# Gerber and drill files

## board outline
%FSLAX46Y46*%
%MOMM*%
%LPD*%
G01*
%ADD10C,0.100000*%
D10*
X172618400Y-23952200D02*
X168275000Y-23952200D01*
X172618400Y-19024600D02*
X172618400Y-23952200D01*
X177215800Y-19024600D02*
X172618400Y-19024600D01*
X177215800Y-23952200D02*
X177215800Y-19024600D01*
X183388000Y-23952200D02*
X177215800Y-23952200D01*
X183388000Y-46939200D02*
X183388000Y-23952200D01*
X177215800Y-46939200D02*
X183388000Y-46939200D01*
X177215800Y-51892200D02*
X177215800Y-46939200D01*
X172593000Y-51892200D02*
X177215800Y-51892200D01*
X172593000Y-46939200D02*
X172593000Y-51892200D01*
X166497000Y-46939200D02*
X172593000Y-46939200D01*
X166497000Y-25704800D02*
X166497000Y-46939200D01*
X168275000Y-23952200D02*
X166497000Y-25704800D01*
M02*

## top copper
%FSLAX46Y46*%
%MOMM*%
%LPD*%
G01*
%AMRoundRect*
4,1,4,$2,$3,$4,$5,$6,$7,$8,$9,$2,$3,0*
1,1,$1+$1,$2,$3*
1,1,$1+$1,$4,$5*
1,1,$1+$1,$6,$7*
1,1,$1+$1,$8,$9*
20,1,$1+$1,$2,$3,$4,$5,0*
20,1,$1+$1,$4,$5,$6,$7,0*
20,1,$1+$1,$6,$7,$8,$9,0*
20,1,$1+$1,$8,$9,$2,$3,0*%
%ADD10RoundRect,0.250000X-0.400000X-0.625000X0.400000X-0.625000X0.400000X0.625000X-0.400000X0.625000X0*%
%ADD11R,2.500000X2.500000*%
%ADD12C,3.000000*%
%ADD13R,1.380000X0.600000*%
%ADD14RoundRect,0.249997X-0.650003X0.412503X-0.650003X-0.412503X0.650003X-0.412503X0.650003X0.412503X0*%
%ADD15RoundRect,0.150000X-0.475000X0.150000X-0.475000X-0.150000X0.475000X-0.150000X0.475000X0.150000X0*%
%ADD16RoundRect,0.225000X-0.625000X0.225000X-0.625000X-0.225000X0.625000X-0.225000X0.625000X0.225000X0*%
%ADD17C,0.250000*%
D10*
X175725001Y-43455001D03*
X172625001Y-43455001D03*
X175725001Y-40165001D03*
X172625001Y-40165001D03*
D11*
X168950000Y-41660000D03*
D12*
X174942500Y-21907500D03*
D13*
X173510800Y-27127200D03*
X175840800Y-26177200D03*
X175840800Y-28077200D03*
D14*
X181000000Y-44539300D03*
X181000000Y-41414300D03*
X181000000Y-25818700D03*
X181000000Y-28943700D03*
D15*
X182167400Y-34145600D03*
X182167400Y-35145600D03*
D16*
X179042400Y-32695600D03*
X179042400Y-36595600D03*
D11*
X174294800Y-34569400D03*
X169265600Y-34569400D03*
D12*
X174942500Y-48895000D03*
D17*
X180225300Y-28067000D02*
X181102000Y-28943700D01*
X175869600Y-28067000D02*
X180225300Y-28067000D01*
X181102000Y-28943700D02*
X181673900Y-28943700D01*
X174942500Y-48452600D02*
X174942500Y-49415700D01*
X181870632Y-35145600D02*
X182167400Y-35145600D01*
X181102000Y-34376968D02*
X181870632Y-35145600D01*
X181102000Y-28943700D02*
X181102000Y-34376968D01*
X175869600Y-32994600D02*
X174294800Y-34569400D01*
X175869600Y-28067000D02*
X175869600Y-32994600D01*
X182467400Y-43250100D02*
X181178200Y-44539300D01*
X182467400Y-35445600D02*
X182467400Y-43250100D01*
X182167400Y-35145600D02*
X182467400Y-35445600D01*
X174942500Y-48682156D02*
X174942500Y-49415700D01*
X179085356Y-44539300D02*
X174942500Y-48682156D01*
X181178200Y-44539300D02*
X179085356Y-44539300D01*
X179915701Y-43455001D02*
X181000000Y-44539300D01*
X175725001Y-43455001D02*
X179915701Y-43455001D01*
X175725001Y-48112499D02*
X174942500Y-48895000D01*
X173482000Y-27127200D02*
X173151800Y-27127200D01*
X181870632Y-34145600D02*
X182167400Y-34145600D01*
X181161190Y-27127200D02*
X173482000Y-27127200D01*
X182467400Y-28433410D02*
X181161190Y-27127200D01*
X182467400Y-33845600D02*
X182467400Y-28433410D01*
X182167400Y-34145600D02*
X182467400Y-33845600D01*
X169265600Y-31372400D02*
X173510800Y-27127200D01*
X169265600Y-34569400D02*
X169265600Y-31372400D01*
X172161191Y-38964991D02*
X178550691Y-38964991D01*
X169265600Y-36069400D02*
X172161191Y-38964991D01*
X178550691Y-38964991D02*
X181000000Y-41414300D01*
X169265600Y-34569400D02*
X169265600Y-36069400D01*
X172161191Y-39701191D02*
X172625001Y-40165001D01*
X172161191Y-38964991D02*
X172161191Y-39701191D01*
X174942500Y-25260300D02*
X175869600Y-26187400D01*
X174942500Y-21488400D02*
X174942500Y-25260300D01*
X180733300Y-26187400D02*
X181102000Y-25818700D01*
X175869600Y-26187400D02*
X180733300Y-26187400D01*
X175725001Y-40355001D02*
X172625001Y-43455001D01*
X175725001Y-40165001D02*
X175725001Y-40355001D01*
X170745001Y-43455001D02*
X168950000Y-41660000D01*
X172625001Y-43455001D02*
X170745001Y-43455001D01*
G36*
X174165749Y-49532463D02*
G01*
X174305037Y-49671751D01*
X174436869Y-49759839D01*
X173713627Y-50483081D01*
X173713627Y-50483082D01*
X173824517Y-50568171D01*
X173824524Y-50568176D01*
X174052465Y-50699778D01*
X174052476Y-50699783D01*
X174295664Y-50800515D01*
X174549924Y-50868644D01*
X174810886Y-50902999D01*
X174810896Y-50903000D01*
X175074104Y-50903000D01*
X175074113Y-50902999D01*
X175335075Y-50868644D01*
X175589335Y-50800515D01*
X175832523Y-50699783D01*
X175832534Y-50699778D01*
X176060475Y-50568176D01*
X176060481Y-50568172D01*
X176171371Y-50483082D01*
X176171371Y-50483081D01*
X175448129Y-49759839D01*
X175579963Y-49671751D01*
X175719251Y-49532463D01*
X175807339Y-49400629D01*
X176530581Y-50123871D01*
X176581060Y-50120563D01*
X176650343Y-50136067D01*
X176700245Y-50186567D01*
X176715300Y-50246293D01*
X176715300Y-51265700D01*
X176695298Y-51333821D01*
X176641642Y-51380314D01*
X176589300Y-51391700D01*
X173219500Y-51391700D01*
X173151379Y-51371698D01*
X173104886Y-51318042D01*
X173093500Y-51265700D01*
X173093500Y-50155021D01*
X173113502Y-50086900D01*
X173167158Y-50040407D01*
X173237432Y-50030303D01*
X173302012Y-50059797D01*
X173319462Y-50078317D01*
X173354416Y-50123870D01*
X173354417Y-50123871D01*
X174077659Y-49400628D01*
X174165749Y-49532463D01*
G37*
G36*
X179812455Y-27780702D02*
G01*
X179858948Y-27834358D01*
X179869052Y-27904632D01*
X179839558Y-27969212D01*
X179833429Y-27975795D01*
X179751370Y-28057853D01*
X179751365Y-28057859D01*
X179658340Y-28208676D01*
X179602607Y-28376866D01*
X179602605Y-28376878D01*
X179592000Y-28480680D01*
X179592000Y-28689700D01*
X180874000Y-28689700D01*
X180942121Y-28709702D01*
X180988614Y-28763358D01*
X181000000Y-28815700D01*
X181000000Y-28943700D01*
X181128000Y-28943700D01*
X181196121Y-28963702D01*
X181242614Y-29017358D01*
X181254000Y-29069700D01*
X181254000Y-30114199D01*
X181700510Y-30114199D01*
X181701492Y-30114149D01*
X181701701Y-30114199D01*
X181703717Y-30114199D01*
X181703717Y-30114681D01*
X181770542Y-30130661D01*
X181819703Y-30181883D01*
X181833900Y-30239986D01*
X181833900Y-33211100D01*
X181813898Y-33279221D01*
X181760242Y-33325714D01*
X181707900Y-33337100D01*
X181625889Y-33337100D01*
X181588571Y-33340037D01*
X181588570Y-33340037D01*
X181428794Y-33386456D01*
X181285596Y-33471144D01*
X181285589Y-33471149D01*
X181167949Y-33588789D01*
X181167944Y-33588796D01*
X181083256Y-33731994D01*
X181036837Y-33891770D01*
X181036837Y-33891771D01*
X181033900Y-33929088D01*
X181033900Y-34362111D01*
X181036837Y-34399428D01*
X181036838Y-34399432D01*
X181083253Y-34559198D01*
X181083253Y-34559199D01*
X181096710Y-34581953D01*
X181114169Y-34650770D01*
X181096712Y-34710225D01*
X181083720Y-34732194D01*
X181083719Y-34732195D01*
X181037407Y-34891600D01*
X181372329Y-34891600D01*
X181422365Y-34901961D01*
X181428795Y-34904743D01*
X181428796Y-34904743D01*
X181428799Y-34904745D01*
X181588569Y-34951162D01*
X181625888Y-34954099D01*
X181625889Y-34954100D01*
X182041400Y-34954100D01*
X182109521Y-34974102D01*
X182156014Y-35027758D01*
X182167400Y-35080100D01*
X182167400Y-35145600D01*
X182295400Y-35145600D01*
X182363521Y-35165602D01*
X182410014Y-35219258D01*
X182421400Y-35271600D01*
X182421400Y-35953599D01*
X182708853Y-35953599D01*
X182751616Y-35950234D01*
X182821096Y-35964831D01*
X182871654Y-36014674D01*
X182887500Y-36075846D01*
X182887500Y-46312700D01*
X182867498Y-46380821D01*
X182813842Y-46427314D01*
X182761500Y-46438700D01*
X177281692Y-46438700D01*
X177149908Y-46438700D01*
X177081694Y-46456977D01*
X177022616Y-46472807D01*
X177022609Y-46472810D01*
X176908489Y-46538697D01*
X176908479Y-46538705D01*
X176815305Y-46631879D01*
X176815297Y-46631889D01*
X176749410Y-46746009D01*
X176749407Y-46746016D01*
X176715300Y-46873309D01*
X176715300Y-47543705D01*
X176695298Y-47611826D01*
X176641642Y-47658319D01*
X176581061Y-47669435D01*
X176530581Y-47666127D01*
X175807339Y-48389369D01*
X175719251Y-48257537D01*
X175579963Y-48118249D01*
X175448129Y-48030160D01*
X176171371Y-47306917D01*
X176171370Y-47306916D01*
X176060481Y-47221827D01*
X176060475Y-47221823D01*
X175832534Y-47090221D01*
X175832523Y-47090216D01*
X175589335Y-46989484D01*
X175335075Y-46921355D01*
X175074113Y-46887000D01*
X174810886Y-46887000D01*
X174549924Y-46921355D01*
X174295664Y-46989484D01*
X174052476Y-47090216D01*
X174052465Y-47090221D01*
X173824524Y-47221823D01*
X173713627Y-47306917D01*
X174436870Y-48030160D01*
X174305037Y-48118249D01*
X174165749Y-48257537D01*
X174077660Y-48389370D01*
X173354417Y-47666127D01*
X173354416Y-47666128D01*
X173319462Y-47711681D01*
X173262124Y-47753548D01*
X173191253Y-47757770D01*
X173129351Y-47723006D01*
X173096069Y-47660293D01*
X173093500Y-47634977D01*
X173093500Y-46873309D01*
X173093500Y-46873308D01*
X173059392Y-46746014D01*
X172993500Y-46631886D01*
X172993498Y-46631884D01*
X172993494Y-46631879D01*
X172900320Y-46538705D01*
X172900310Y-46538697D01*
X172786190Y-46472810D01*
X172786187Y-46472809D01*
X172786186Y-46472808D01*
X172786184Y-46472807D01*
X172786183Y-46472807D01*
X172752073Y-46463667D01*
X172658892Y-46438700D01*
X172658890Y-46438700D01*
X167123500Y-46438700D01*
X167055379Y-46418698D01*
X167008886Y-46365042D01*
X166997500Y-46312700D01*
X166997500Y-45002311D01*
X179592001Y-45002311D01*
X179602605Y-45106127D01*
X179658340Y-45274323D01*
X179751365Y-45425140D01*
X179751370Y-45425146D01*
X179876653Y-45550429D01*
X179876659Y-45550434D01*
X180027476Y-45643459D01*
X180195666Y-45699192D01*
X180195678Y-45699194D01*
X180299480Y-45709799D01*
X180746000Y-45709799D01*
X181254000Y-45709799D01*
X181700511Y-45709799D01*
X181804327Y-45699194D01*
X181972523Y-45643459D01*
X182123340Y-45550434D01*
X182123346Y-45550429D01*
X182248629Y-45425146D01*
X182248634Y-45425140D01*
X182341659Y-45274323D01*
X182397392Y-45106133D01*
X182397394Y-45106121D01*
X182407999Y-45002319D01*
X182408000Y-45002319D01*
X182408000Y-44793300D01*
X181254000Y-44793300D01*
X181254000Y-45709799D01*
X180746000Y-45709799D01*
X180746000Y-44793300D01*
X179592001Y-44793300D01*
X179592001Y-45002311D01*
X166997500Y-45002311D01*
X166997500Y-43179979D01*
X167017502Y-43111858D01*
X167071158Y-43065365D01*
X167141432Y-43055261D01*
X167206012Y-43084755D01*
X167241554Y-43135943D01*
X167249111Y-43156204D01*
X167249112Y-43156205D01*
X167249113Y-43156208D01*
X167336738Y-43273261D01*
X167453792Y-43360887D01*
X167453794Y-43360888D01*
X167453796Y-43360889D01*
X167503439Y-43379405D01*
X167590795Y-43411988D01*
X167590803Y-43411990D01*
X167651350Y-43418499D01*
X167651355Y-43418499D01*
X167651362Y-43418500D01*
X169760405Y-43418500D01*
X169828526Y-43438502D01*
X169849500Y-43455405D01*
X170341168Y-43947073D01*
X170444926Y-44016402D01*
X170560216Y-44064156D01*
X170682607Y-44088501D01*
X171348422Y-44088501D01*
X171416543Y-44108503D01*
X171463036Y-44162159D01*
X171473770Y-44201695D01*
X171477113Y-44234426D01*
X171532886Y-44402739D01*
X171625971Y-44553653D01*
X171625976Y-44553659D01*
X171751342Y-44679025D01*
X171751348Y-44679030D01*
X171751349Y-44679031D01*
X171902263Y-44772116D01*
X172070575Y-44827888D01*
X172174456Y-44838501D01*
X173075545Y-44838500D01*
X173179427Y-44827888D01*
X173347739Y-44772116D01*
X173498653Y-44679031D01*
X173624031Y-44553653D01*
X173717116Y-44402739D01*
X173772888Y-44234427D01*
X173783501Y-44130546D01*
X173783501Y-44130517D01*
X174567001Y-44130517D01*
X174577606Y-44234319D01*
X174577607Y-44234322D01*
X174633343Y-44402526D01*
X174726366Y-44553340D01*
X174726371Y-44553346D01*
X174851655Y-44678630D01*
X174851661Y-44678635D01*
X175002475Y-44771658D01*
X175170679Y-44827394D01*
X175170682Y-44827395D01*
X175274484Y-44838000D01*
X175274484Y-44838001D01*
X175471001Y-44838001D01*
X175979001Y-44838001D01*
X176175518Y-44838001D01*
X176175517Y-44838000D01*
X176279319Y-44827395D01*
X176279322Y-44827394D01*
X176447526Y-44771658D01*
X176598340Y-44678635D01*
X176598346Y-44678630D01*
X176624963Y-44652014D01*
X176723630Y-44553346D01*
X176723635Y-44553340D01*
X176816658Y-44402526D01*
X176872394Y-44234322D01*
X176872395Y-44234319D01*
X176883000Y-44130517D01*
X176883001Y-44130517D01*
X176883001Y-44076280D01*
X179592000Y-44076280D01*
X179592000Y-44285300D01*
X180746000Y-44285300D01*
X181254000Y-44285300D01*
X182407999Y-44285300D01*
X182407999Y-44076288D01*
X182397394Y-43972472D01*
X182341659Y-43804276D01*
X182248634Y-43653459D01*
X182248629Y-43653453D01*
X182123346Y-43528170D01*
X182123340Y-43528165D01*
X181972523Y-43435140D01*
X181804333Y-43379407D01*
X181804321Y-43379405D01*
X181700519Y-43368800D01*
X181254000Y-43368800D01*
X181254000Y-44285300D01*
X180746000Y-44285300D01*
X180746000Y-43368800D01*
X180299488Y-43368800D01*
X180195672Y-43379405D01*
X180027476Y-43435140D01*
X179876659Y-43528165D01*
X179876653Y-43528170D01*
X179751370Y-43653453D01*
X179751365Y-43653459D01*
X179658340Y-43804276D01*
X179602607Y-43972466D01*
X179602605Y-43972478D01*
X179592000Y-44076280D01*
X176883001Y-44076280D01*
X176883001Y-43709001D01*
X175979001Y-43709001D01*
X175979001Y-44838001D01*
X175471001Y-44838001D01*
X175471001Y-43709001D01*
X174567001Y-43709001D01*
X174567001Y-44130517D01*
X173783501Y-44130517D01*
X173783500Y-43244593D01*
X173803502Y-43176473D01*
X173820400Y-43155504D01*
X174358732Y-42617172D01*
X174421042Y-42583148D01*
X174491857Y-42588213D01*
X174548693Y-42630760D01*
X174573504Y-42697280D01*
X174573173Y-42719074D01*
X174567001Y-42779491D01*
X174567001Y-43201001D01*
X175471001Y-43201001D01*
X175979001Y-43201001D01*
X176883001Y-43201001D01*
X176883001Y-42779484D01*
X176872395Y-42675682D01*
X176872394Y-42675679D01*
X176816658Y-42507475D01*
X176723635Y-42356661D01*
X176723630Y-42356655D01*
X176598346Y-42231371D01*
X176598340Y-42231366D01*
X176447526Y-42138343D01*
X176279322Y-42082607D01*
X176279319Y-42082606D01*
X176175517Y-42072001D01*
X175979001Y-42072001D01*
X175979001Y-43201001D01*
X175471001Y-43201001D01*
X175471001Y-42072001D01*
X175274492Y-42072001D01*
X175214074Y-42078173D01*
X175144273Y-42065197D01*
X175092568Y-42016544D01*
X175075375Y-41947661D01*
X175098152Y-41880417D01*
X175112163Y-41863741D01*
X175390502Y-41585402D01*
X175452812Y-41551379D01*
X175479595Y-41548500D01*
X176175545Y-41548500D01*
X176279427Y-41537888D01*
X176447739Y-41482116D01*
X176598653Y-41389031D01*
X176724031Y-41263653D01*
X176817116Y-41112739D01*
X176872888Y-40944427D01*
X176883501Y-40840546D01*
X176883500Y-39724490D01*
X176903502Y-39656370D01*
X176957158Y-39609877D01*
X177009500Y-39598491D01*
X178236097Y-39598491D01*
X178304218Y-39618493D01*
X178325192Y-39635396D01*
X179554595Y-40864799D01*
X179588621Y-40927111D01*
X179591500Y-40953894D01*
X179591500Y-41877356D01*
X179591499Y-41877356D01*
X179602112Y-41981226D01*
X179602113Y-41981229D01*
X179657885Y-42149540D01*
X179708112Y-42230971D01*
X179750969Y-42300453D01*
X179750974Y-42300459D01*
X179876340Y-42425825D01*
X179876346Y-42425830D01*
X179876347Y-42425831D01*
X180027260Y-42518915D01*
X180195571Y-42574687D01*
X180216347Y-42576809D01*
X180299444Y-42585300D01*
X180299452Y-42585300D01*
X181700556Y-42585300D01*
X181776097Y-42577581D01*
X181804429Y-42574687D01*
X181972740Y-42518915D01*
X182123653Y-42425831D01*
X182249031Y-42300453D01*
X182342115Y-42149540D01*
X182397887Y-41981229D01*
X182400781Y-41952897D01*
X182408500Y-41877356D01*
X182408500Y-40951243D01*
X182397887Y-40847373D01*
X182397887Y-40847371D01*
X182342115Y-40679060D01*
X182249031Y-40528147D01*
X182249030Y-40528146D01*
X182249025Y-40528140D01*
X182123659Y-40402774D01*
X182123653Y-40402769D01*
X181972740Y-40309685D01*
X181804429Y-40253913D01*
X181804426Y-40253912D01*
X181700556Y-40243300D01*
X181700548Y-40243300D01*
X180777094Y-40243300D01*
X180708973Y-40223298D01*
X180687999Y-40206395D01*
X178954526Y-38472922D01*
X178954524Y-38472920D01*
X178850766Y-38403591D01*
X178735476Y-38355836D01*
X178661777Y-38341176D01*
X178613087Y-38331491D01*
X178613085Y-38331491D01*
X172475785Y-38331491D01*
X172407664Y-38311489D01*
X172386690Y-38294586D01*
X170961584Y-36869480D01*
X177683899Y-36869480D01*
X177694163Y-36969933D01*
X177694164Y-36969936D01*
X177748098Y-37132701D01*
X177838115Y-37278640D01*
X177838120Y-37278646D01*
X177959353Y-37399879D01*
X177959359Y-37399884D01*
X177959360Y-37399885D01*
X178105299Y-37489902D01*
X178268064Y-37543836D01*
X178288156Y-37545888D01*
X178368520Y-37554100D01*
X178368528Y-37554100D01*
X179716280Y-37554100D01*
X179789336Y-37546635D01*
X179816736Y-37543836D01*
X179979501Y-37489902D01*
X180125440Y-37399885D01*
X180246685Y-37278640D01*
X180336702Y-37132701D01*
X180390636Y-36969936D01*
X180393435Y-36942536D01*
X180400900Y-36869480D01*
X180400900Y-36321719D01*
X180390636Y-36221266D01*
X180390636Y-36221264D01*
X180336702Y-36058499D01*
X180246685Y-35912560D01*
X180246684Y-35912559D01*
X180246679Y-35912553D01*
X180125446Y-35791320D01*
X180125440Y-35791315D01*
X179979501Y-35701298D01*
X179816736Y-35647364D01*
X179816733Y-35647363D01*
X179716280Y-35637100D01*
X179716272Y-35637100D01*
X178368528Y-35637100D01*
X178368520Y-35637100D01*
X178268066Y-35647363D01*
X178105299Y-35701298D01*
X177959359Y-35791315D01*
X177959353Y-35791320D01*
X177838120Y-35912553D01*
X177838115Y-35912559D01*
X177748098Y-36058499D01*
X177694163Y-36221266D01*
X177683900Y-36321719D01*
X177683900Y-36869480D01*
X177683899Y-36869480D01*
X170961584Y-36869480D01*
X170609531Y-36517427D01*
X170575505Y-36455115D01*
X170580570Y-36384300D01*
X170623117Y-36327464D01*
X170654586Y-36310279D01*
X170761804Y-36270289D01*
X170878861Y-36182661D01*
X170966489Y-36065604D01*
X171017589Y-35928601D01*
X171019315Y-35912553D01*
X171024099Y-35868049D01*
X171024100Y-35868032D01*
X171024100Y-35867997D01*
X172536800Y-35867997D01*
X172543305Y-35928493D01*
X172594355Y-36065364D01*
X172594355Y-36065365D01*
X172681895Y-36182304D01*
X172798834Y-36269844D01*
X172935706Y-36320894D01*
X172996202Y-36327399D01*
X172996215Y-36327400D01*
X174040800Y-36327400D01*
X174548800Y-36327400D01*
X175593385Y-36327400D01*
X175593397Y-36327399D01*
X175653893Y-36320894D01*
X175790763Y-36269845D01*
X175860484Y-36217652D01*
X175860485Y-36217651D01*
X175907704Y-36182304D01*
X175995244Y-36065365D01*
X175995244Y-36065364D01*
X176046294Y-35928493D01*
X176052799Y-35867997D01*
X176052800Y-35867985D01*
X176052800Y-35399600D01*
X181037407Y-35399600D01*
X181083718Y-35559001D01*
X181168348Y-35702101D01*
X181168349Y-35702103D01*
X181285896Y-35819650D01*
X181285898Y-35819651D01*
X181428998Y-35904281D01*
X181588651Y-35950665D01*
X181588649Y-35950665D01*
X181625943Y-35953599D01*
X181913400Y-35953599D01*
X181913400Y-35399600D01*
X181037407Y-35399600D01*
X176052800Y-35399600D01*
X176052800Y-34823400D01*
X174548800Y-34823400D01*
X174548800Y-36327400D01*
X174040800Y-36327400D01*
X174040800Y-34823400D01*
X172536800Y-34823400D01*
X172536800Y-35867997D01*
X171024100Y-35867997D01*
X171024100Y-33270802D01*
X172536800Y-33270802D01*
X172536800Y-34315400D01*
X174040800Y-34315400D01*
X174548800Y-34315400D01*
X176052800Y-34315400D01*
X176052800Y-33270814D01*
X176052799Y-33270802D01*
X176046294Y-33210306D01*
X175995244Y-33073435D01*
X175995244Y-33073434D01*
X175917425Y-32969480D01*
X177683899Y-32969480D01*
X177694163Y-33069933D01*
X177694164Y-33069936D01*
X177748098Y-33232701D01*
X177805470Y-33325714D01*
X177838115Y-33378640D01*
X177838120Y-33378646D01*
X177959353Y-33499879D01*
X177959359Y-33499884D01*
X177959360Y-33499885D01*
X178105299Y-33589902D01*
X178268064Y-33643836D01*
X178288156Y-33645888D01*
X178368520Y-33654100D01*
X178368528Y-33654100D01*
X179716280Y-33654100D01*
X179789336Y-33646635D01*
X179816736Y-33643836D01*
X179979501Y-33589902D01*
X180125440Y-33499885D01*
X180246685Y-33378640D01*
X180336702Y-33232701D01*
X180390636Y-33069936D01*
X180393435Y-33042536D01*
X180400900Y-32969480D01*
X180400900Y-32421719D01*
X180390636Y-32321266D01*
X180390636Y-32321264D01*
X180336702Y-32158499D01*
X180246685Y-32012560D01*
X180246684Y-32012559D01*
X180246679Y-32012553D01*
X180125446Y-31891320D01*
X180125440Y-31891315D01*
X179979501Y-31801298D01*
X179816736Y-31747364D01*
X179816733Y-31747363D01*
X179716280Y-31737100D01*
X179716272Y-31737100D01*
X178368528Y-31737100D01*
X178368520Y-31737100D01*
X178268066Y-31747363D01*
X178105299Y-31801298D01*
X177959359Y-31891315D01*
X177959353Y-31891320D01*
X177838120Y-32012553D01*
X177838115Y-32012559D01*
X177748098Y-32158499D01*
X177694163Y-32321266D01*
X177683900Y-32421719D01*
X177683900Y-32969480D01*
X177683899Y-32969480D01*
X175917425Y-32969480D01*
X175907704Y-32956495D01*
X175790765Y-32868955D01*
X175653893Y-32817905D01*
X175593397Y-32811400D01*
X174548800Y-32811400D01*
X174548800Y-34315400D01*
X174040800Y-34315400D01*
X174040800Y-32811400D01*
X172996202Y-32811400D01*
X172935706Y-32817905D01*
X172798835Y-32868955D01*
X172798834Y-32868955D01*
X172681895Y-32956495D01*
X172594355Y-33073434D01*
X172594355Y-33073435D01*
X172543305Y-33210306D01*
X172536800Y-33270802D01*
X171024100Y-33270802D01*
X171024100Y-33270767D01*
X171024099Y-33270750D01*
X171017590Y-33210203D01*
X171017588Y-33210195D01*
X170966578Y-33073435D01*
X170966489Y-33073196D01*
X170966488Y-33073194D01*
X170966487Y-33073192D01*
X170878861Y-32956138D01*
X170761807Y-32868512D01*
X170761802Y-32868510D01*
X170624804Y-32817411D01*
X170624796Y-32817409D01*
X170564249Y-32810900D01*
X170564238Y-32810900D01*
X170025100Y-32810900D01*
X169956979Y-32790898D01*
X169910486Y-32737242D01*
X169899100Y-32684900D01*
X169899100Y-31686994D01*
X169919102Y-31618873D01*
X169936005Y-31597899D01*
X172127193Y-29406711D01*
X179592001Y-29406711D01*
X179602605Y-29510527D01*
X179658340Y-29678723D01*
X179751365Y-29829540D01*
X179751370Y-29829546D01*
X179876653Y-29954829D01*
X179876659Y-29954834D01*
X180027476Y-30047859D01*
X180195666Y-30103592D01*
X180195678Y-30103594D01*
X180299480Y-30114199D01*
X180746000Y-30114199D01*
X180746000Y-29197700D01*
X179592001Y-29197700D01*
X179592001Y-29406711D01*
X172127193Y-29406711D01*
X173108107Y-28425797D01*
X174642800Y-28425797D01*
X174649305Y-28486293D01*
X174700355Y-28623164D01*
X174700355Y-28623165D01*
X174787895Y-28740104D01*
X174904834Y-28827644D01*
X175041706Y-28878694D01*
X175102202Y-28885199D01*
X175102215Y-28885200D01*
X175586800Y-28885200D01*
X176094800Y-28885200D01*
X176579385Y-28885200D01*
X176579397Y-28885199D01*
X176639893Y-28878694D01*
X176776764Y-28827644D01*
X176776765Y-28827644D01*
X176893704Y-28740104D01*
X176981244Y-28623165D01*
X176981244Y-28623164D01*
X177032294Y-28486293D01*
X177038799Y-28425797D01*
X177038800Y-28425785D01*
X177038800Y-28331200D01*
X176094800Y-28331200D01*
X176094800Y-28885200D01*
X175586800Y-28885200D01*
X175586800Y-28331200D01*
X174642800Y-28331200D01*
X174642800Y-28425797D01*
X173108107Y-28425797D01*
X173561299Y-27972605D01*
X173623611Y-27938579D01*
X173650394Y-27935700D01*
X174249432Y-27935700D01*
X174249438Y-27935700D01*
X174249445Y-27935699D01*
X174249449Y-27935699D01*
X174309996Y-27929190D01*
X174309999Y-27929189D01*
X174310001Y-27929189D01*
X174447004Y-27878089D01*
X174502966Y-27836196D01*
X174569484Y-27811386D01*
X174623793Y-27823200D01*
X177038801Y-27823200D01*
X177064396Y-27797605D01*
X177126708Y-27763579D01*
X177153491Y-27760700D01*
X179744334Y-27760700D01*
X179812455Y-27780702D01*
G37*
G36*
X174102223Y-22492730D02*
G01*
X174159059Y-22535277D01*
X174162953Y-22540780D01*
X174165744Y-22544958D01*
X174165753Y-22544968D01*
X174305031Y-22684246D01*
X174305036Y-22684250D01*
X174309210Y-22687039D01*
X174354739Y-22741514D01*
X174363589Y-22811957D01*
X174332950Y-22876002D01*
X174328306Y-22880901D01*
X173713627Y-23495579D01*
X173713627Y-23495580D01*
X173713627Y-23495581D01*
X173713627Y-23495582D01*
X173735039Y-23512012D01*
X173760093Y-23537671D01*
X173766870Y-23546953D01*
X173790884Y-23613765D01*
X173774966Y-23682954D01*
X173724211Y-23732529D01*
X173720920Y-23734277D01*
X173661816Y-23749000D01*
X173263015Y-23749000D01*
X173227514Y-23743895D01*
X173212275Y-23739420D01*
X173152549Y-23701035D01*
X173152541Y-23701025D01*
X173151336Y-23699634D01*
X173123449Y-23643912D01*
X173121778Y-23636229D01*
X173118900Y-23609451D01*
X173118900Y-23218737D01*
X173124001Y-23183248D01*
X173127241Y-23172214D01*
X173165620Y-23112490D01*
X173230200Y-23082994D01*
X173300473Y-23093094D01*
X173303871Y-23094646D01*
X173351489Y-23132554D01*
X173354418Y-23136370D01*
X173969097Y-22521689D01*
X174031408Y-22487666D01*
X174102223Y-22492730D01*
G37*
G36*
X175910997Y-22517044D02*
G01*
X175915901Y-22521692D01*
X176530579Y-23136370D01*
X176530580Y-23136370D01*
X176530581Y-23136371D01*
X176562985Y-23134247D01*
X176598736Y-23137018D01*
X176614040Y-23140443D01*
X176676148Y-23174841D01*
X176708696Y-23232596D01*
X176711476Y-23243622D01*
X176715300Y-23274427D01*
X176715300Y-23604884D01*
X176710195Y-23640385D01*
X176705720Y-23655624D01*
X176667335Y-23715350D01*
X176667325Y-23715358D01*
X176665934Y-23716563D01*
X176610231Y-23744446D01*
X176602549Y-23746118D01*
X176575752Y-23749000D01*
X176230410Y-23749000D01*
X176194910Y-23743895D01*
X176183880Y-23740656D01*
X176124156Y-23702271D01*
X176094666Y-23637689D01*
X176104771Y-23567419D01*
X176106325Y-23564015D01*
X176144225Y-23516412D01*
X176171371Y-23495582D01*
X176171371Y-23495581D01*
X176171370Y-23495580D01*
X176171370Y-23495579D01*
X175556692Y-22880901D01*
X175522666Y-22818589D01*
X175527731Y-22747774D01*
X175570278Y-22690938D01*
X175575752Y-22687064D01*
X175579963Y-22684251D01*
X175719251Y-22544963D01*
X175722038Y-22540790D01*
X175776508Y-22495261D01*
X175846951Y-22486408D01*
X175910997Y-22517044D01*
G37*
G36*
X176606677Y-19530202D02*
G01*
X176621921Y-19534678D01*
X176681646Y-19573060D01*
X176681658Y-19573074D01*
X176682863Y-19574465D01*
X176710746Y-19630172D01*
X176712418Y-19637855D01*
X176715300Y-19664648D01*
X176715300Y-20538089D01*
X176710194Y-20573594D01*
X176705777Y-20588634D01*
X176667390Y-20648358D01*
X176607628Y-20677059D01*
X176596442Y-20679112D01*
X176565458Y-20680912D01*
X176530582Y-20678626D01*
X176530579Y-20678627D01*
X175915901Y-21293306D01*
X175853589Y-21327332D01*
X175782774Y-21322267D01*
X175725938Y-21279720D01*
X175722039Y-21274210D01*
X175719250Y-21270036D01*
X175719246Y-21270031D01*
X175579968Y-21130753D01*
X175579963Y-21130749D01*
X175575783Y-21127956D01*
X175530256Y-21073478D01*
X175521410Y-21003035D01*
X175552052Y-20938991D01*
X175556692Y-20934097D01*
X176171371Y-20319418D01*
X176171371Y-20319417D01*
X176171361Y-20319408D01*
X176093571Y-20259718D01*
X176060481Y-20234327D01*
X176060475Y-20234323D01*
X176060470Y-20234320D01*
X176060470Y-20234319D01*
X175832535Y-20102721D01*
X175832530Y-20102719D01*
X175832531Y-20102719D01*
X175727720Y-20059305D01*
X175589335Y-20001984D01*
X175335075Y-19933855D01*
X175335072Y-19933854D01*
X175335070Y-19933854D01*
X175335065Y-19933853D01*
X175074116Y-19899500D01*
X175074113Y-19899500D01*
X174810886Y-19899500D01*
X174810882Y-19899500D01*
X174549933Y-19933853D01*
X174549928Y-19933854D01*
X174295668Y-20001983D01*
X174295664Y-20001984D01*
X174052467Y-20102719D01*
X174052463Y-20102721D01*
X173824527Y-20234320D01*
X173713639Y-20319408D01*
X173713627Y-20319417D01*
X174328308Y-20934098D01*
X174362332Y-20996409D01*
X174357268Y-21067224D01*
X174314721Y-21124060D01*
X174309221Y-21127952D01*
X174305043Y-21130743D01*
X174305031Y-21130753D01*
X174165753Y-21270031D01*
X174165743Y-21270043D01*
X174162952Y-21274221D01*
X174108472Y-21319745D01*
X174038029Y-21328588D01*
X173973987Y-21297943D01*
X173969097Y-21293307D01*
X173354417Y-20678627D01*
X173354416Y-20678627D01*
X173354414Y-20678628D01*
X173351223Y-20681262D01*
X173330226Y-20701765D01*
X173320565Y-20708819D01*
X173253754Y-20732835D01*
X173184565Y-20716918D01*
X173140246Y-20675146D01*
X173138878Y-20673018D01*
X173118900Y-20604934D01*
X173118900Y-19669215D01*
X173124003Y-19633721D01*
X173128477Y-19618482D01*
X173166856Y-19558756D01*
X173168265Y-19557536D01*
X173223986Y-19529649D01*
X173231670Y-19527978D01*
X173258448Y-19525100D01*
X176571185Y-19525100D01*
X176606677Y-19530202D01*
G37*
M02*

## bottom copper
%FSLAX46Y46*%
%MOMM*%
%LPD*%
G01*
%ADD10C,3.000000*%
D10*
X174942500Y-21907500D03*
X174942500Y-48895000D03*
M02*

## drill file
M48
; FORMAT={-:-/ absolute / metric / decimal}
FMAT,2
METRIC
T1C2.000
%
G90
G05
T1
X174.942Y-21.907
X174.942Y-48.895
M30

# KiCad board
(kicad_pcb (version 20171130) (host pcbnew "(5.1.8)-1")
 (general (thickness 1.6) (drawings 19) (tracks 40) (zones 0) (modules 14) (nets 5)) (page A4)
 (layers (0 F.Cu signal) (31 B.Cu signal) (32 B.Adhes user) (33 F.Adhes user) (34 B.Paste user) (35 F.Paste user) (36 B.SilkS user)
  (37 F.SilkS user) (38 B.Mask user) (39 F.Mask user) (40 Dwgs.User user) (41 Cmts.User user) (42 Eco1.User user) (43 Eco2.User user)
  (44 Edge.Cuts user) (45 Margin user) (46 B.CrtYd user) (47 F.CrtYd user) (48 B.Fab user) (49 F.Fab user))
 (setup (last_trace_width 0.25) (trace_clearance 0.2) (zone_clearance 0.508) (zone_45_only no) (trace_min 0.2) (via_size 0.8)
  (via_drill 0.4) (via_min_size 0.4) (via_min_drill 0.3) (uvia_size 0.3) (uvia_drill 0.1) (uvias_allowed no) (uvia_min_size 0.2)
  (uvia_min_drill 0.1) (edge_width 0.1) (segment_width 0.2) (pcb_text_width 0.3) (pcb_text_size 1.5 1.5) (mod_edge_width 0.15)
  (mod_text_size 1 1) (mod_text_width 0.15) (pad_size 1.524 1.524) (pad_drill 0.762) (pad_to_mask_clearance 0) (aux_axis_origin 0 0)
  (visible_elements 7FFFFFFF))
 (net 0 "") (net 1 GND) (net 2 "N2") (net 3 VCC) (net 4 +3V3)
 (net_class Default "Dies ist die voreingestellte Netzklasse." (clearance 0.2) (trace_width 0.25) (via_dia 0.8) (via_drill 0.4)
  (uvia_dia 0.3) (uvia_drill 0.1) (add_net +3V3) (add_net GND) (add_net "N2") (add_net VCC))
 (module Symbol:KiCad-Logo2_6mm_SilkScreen (layer B.Cu) (at 169.7 35.36 270)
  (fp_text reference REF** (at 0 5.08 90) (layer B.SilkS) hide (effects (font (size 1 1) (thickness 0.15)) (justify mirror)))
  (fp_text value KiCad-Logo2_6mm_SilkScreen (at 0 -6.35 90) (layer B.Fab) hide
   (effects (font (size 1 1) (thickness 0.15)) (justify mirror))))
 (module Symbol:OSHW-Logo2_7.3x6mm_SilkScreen (layer B.Cu) (at 178.48 35.75 270)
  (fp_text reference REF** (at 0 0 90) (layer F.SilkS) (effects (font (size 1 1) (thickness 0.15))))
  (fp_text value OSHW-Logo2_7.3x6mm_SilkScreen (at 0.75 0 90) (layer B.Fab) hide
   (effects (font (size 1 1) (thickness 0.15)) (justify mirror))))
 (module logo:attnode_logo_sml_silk (layer F.Cu) (at 169.78 25.8)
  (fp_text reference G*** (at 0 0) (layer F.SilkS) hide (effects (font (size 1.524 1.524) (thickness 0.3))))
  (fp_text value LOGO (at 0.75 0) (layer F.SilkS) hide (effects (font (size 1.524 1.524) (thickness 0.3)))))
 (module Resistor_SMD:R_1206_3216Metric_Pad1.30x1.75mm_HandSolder (layer F.Cu) (at 174.175001 43.455001)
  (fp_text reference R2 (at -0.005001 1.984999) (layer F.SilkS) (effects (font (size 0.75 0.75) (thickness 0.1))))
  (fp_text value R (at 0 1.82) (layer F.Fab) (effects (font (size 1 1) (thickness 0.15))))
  (pad 2 smd roundrect (at 1.55 0) (size 1.3 1.75) (layers F.Cu F.Paste F.Mask) (roundrect_rratio 0.1923076923076923) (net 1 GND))
  (pad 1 smd roundrect (at -1.55 0) (size 1.3 1.75) (layers F.Cu F.Paste F.Mask) (roundrect_rratio 0.1923076923076923) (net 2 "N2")))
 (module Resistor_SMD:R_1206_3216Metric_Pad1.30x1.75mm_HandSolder (layer F.Cu) (at 174.175001 40.165001)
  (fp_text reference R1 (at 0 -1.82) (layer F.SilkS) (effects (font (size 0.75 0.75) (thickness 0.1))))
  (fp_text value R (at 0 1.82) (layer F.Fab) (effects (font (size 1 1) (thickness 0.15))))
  (pad 2 smd roundrect (at 1.55 0) (size 1.3 1.75) (layers F.Cu F.Paste F.Mask) (roundrect_rratio 0.1923076923076923) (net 2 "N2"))
  (pad 1 smd roundrect (at -1.55 0) (size 1.3 1.75) (layers F.Cu F.Paste F.Mask) (roundrect_rratio 0.1923076923076923) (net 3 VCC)))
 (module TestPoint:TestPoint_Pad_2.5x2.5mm (layer F.Cu) (at 168.95 41.66)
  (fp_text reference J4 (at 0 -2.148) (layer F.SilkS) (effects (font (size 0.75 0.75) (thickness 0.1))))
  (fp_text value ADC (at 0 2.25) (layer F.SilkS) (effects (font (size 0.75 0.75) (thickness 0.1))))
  (pad 1 smd rect (at 0 0) (size 2.5 2.5) (layers F.Cu F.Mask) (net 2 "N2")))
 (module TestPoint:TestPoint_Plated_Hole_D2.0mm (layer F.Cu) (at 174.9425 21.9075)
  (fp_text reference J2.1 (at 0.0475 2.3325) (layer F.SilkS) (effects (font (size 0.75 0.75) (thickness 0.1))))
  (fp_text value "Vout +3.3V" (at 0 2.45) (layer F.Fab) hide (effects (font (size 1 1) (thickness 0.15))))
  (pad 1 thru_hole circle (at 0 0) (size 3 3) (drill 2) (layers *.Cu *.Mask) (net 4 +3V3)))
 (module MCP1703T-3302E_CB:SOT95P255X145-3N (layer F.Cu) (at 174.6758 27.1272 180)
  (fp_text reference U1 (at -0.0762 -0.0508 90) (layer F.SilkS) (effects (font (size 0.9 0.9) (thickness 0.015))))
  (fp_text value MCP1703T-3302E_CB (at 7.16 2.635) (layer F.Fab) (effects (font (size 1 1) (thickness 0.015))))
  (pad 3 smd rect (at 1.165 0 180) (size 1.38 0.6) (layers F.Cu F.Paste F.Mask) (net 3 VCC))
  (pad 2 smd rect (at -1.165 0.95 180) (size 1.38 0.6) (layers F.Cu F.Paste F.Mask) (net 4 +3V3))
  (pad 1 smd rect (at -1.165 -0.95 180) (size 1.38 0.6) (layers F.Cu F.Paste F.Mask) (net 1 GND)))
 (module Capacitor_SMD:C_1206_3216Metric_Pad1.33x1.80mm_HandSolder (layer F.Cu) (at 181 42.9768 270)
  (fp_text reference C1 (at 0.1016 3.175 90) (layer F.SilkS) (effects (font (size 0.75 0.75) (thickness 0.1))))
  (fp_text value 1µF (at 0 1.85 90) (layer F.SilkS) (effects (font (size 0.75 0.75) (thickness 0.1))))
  (pad 2 smd roundrect (at 1.5625 0 270) (size 1.325 1.8) (layers F.Cu F.Paste F.Mask) (roundrect_rratio 0.1886769811320755) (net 1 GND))
  (pad 1 smd roundrect (at -1.5625 0 270) (size 1.325 1.8) (layers F.Cu F.Paste F.Mask) (roundrect_rratio 0.1886769811320755) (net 3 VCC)))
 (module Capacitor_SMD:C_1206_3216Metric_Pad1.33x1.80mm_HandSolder (layer F.Cu) (at 181 27.3812 270)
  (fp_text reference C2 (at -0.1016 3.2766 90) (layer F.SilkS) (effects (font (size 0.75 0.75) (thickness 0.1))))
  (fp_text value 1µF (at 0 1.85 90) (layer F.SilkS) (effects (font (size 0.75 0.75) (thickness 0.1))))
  (pad 1 smd roundrect (at -1.5625 0 270) (size 1.325 1.8) (layers F.Cu F.Paste F.Mask) (roundrect_rratio 0.1886769811320755) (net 4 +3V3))
  (pad 2 smd roundrect (at 1.5625 0 270) (size 1.325 1.8) (layers F.Cu F.Paste F.Mask) (roundrect_rratio 0.1886769811320755) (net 1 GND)))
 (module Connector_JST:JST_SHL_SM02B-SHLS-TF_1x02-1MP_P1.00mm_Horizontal (layer F.Cu) (at 180.4924 34.6456 270)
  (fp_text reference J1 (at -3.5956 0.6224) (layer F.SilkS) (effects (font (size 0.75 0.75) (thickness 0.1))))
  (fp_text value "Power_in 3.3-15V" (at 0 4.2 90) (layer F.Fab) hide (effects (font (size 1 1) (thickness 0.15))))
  (pad 1 smd roundrect (at -0.5 -1.675 270) (size 0.6 1.25) (layers F.Cu F.Paste F.Mask) (roundrect_rratio 0.25) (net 3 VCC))
  (pad 2 smd roundrect (at 0.5 -1.675 270) (size 0.6 1.25) (layers F.Cu F.Paste F.Mask) (roundrect_rratio 0.25) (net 1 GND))
  (pad MP smd roundrect (at -1.95 1.45 270) (size 0.9 1.7) (layers F.Cu F.Paste F.Mask) (roundrect_rratio 0.25))
  (pad MP smd roundrect (at 1.95 1.45 270) (size 0.9 1.7) (layers F.Cu F.Paste F.Mask) (roundrect_rratio 0.25)))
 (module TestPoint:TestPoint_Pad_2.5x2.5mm (layer F.Cu) (at 174.2948 34.5694)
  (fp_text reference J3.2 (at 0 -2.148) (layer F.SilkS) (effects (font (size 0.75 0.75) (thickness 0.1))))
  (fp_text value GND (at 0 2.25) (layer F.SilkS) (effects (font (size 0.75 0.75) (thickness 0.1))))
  (pad 1 smd rect (at 0 0) (size 2.5 2.5) (layers F.Cu F.Mask) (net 1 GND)))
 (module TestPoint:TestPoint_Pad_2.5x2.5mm (layer F.Cu) (at 169.2656 34.5694)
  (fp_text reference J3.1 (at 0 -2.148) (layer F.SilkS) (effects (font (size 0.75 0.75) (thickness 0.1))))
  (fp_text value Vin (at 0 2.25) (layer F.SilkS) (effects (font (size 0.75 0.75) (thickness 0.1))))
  (pad 1 smd rect (at 0 0) (size 2.5 2.5) (layers F.Cu F.Mask) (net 3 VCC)))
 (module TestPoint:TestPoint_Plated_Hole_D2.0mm (layer F.Cu) (at 174.9425 48.895)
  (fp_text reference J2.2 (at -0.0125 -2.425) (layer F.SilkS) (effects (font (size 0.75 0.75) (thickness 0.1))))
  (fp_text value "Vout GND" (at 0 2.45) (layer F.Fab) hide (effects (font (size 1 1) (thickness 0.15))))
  (pad 1 thru_hole circle (at 0 0) (size 3 3) (drill 2) (layers *.Cu *.Mask) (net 1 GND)))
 (gr_line (start 172.6184 23.9522) (end 168.275 23.9522) (layer Edge.Cuts) (width 0.1))
 (gr_line (start 172.6184 19.0246) (end 172.6184 23.9522) (layer Edge.Cuts) (width 0.1))
 (gr_line (start 177.2158 19.0246) (end 172.6184 19.0246) (layer Edge.Cuts) (width 0.1))
 (gr_line (start 177.2158 23.9522) (end 177.2158 19.0246) (layer Edge.Cuts) (width 0.1))
 (gr_line (start 183.388 23.9522) (end 177.2158 23.9522) (layer Edge.Cuts) (width 0.1))
 (gr_line (start 183.388 46.9392) (end 183.388 23.9522) (layer Edge.Cuts) (width 0.1))
 (gr_line (start 177.2158 46.9392) (end 183.388 46.9392) (layer Edge.Cuts) (width 0.1))
 (gr_line (start 177.2158 51.8922) (end 177.2158 46.9392) (layer Edge.Cuts) (width 0.1))
 (gr_line (start 172.593 51.8922) (end 177.2158 51.8922) (layer Edge.Cuts) (width 0.1))
 (gr_line (start 172.593 46.9392) (end 172.593 51.8922) (layer Edge.Cuts) (width 0.1))
 (gr_line (start 166.497 46.9392) (end 172.593 46.9392) (layer Edge.Cuts) (width 0.1))
 (gr_line (start 166.497 25.7048) (end 166.497 46.9392) (layer Edge.Cuts) (width 0.1))
 (gr_line (start 168.275 23.9522) (end 166.497 25.7048) (layer Edge.Cuts) (width 0.1))
 (segment (start 180.2253 28.067) (end 181.102 28.9437) (width 0.25) (layer F.Cu) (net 1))
 (segment (start 175.8696 28.067) (end 180.2253 28.067) (width 0.25) (layer F.Cu) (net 1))
 (segment (start 181.102 28.9437) (end 181.6739 28.9437) (width 0.25) (layer F.Cu) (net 1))
 (segment (start 174.9425 48.4526) (end 174.9425 49.4157) (width 0.25) (layer F.Cu) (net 1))
 (segment (start 181.870632 35.1456) (end 182.1674 35.1456) (width 0.25) (layer F.Cu) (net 1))
 (segment (start 181.102 34.376968) (end 181.870632 35.1456) (width 0.25) (layer F.Cu) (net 1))
 (segment (start 181.102 28.9437) (end 181.102 34.376968) (width 0.25) (layer F.Cu) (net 1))
 (segment (start 175.8696 32.9946) (end 174.2948 34.5694) (width 0.25) (layer F.Cu) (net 1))
 (segment (start 175.8696 28.067) (end 175.8696 32.9946) (width 0.25) (layer F.Cu) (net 1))
 (segment (start 182.4674 43.2501) (end 181.1782 44.5393) (width 0.25) (layer F.Cu) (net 1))
 (segment (start 182.4674 35.4456) (end 182.4674 43.2501) (width 0.25) (layer F.Cu) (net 1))
 (segment (start 182.1674 35.1456) (end 182.4674 35.4456) (width 0.25) (layer F.Cu) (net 1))
 (segment (start 174.9425 48.682156) (end 174.9425 49.4157) (width 0.25) (layer F.Cu) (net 1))
 (segment (start 179.085356 44.5393) (end 174.9425 48.682156) (width 0.25) (layer F.Cu) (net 1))
 (segment (start 181.1782 44.5393) (end 179.085356 44.5393) (width 0.25) (layer F.Cu) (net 1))
 (segment (start 179.915701 43.455001) (end 181 44.5393) (width 0.25) (layer F.Cu) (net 1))
 (segment (start 175.725001 43.455001) (end 179.915701 43.455001) (width 0.25) (layer F.Cu) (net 1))
 (segment (start 175.725001 48.112499) (end 174.9425 48.895) (width 0.25) (layer F.Cu) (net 1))
 (segment (start 173.482 27.1272) (end 173.1518 27.1272) (width 0.25) (layer F.Cu) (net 3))
 (segment (start 181.870632 34.1456) (end 182.1674 34.1456) (width 0.25) (layer F.Cu) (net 3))
 (segment (start 181.16119 27.1272) (end 173.482 27.1272) (width 0.25) (layer F.Cu) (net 3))
 (segment (start 182.4674 28.43341) (end 181.16119 27.1272) (width 0.25) (layer F.Cu) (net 3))
 (segment (start 182.4674 33.8456) (end 182.4674 28.43341) (width 0.25) (layer F.Cu) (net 3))
 (segment (start 182.1674 34.1456) (end 182.4674 33.8456) (width 0.25) (layer F.Cu) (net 3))
 (segment (start 169.2656 31.3724) (end 173.5108 27.1272) (width 0.25) (layer F.Cu) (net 3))
 (segment (start 169.2656 34.5694) (end 169.2656 31.3724) (width 0.25) (layer F.Cu) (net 3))
 (segment (start 172.161191 38.964991) (end 178.550691 38.964991) (width 0.25) (layer F.Cu) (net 3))
 (segment (start 169.2656 36.0694) (end 172.161191 38.964991) (width 0.25) (layer F.Cu) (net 3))
 (segment (start 178.550691 38.964991) (end 181 41.4143) (width 0.25) (layer F.Cu) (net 3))
 (segment (start 169.2656 34.5694) (end 169.2656 36.0694) (width 0.25) (layer F.Cu) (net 3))
 (segment (start 172.161191 39.701191) (end 172.625001 40.165001) (width 0.25) (layer F.Cu) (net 3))
 (segment (start 172.161191 38.964991) (end 172.161191 39.701191) (width 0.25) (layer F.Cu) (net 3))
 (segment (start 174.9425 25.2603) (end 175.8696 26.1874) (width 0.25) (layer F.Cu) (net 4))
 (segment (start 174.9425 21.4884) (end 174.9425 25.2603) (width 0.25) (layer F.Cu) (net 4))
 (segment (start 180.7333 26.1874) (end 181.102 25.8187) (width 0.25) (layer F.Cu) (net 4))
 (segment (start 175.8696 26.1874) (end 180.7333 26.1874) (width 0.25) (layer F.Cu) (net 4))
 (segment (start 175.725001 40.355001) (end 172.625001 43.455001) (width 0.25) (layer F.Cu) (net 2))
 (segment (start 175.725001 40.165001) (end 175.725001 40.355001) (width 0.25) (layer F.Cu) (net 2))
 (segment (start 170.745001 43.455001) (end 168.95 41.66) (width 0.25) (layer F.Cu) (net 2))
 (segment (start 172.625001 43.455001) (end 170.745001 43.455001) (width 0.25) (layer F.Cu) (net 2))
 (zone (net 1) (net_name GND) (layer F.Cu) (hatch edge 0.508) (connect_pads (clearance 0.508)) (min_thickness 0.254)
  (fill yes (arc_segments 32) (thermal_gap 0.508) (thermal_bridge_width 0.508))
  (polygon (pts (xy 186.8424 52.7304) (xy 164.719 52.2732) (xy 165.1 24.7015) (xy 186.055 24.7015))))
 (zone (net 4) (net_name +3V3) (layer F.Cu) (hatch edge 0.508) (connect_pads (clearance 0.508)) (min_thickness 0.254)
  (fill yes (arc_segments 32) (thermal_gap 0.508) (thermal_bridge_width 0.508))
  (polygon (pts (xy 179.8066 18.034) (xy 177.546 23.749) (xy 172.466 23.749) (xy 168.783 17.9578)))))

